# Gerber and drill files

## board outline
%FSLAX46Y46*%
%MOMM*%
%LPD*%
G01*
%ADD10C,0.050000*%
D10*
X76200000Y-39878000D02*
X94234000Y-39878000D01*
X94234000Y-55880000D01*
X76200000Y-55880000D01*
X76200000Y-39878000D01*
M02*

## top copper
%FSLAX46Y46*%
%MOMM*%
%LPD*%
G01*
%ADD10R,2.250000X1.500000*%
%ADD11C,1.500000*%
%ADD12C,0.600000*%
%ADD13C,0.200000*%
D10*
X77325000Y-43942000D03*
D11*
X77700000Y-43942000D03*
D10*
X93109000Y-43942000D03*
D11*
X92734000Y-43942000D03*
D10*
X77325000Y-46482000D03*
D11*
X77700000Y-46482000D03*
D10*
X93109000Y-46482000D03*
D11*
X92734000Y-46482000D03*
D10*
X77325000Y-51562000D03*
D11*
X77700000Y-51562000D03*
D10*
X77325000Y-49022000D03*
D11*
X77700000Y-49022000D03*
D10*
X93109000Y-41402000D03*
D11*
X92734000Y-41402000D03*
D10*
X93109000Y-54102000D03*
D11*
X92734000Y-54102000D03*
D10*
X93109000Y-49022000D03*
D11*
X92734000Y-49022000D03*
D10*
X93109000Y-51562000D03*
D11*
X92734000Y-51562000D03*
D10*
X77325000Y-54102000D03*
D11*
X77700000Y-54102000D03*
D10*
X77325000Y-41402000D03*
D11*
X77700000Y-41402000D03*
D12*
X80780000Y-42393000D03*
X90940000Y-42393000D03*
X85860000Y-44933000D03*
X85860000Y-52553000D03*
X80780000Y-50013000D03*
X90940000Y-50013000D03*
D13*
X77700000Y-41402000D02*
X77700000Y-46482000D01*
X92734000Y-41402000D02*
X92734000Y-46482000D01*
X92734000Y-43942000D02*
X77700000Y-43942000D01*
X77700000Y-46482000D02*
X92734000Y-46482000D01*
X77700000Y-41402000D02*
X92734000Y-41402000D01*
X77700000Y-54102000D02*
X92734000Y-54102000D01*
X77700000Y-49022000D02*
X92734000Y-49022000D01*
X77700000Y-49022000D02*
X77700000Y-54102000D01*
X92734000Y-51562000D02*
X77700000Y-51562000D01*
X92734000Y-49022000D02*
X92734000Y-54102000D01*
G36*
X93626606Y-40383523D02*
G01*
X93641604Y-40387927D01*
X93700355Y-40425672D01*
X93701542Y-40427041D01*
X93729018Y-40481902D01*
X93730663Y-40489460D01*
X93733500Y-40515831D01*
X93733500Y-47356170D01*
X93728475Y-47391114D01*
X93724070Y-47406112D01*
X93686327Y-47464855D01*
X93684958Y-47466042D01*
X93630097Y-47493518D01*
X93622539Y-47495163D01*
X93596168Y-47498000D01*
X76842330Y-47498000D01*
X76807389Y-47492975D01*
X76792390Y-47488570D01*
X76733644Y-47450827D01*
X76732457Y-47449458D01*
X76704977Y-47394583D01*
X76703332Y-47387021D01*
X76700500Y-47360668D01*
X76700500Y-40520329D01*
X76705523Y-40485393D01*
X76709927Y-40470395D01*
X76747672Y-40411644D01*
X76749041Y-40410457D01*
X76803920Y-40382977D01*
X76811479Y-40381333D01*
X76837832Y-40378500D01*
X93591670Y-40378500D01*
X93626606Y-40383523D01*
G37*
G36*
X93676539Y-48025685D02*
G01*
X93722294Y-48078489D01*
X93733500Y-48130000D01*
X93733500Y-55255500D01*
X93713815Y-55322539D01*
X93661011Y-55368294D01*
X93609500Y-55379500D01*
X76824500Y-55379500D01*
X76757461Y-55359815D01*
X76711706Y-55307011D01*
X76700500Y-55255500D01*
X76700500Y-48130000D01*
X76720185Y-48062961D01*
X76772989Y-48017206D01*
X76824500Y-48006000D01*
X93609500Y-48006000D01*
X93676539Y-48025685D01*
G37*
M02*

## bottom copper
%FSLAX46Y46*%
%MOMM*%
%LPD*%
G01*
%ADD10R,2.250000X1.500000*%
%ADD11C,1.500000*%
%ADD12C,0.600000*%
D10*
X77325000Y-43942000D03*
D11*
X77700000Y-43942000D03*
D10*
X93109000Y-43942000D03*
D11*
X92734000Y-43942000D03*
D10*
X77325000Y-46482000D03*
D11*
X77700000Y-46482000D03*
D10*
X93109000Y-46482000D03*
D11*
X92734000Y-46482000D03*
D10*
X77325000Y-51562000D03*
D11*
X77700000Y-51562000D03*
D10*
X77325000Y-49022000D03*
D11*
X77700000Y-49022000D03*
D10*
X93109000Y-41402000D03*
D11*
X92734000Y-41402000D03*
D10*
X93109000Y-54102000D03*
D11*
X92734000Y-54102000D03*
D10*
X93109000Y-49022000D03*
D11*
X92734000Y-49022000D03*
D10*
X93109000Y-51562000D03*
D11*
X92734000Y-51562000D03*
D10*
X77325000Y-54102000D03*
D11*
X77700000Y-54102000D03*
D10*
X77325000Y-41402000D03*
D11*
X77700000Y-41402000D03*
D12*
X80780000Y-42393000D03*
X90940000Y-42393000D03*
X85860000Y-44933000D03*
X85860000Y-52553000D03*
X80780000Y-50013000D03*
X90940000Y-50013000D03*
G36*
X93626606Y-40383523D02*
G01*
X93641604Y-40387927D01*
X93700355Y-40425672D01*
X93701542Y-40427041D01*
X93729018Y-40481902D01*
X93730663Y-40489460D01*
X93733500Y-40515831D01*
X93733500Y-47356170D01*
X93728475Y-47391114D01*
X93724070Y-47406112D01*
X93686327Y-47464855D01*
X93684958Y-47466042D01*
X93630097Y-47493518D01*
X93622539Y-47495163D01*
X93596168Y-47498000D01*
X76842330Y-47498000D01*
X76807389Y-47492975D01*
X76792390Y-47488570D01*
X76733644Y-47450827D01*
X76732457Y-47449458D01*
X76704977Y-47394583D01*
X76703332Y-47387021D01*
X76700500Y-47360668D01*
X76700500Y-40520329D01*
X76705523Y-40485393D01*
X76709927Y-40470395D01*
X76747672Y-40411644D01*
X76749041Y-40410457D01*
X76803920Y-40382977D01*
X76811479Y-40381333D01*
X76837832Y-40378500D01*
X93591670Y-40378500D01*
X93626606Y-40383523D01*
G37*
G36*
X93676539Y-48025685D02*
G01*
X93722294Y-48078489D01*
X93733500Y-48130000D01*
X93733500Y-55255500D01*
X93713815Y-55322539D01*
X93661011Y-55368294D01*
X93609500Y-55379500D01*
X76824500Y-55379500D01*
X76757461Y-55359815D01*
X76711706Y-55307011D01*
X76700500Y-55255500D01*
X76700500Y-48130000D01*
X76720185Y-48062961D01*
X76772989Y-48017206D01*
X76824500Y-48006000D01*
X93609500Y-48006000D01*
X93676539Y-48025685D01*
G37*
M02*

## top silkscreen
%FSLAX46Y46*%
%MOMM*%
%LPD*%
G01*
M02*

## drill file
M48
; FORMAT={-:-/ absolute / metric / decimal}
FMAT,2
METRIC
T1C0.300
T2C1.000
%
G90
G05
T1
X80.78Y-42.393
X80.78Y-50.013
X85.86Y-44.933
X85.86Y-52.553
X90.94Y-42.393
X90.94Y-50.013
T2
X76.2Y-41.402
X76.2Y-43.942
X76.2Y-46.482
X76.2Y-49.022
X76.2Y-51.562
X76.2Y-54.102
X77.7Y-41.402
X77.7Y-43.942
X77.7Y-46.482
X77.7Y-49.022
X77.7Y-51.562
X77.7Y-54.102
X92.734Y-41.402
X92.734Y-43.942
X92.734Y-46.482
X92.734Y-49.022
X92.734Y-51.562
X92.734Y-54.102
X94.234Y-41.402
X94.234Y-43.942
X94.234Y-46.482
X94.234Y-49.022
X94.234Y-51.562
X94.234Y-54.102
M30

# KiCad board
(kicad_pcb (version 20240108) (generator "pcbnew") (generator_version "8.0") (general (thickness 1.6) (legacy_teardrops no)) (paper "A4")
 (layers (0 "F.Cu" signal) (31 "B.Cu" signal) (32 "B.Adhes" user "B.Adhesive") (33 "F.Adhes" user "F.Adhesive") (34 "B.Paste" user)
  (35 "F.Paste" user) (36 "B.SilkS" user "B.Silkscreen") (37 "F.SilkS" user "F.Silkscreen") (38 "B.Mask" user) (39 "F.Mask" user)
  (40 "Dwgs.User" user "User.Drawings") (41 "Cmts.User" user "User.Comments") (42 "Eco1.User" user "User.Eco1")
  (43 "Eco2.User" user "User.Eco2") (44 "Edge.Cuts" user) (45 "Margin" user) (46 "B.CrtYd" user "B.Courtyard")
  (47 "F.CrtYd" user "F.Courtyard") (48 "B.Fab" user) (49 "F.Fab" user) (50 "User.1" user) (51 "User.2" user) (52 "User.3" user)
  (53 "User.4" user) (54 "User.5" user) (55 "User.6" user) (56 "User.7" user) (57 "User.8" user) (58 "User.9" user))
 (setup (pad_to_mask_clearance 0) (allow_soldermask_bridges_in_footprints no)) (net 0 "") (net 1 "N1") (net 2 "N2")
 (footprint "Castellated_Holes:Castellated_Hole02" (layer "F.Cu") (at 76.2 43.942)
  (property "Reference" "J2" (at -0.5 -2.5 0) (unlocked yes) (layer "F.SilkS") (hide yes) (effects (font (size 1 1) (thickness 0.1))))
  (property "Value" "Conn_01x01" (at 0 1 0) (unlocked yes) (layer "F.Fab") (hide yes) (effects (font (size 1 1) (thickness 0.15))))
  (pad "1" thru_hole rect (at 0 0) (size 2.25 1.5) (drill 1 (offset 1.125 0)) (layers "*.Cu" "*.Mask") (remove_unused_layers no)
   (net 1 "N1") (solder_mask_margin 0.04))
  (pad "1" thru_hole circle (at 1.5 0) (size 1.5 1.5) (drill 1) (layers "*.Cu" "*.Mask") (remove_unused_layers no) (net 1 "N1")
   (solder_mask_margin 0.04)))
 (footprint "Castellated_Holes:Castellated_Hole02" (layer "F.Cu") (at 94.234 43.942 180)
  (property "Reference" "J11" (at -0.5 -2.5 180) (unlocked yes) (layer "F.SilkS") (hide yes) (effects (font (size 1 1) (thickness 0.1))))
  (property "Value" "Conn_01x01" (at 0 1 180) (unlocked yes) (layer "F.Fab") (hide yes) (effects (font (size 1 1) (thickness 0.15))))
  (pad "1" thru_hole rect (at 0 0 180) (size 2.25 1.5) (drill 1 (offset 1.125 0)) (layers "*.Cu" "*.Mask") (remove_unused_layers no)
   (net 1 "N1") (solder_mask_margin 0.04))
  (pad "1" thru_hole circle (at 1.5 0 180) (size 1.5 1.5) (drill 1) (layers "*.Cu" "*.Mask") (remove_unused_layers no) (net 1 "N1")
   (solder_mask_margin 0.04)))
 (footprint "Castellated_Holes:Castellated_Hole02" (layer "F.Cu") (at 76.2 46.482)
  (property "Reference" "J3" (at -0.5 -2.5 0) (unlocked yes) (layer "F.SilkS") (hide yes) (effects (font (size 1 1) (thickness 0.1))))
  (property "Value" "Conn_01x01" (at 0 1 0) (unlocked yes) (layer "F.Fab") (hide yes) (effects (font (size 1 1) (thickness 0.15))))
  (pad "1" thru_hole rect (at 0 0) (size 2.25 1.5) (drill 1 (offset 1.125 0)) (layers "*.Cu" "*.Mask") (remove_unused_layers no)
   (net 1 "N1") (solder_mask_margin 0.04))
  (pad "1" thru_hole circle (at 1.5 0) (size 1.5 1.5) (drill 1) (layers "*.Cu" "*.Mask") (remove_unused_layers no) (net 1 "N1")
   (solder_mask_margin 0.04)))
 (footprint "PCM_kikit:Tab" (layer "F.Cu") (at 92.964 39.624 -90)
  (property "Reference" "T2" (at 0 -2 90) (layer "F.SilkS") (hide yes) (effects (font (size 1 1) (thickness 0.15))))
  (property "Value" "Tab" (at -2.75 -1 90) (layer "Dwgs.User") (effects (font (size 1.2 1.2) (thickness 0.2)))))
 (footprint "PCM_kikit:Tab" (layer "F.Cu") (at 77.47 39.624 -90)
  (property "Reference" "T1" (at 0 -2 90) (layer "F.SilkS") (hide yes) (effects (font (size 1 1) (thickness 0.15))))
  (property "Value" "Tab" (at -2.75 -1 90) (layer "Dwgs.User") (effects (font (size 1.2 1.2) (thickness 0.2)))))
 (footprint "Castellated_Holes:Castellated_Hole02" (layer "F.Cu") (at 94.234 46.482 180)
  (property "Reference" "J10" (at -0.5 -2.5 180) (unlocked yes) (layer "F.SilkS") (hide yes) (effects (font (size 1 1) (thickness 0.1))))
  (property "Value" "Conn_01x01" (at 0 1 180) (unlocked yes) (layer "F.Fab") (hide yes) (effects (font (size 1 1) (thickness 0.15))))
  (pad "1" thru_hole rect (at 0 0 180) (size 2.25 1.5) (drill 1 (offset 1.125 0)) (layers "*.Cu" "*.Mask") (remove_unused_layers no)
   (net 1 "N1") (solder_mask_margin 0.04))
  (pad "1" thru_hole circle (at 1.5 0 180) (size 1.5 1.5) (drill 1) (layers "*.Cu" "*.Mask") (remove_unused_layers no) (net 1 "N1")
   (solder_mask_margin 0.04)))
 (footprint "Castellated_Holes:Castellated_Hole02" (layer "F.Cu") (at 76.2 51.562)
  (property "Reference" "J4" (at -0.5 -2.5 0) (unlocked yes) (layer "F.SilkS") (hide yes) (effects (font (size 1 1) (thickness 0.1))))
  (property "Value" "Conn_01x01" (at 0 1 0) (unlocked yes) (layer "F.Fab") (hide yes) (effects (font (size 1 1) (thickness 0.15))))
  (pad "1" thru_hole rect (at 0 0) (size 2.25 1.5) (drill 1 (offset 1.125 0)) (layers "*.Cu" "*.Mask") (remove_unused_layers no)
   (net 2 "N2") (solder_mask_margin 0.04))
  (pad "1" thru_hole circle (at 1.5 0) (size 1.5 1.5) (drill 1) (layers "*.Cu" "*.Mask") (remove_unused_layers no) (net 2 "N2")
   (solder_mask_margin 0.04)))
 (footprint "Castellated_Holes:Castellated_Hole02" (layer "F.Cu") (at 76.2 49.022)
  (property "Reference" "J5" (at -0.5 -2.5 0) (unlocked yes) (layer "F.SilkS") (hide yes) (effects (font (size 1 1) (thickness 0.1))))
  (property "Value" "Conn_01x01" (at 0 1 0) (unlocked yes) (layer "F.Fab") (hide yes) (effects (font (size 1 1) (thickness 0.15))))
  (pad "1" thru_hole rect (at 0 0) (size 2.25 1.5) (drill 1 (offset 1.125 0)) (layers "*.Cu" "*.Mask") (remove_unused_layers no)
   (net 2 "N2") (solder_mask_margin 0.04))
  (pad "1" thru_hole circle (at 1.5 0) (size 1.5 1.5) (drill 1) (layers "*.Cu" "*.Mask") (remove_unused_layers no) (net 2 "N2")
   (solder_mask_margin 0.04)))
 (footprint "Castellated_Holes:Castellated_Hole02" (layer "F.Cu") (at 94.234 41.402 180)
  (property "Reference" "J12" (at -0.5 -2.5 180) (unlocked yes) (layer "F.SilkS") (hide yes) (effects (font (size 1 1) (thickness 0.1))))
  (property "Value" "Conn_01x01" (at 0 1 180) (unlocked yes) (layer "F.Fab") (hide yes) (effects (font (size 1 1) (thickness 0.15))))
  (pad "1" thru_hole rect (at 0 0 180) (size 2.25 1.5) (drill 1 (offset 1.125 0)) (layers "*.Cu" "*.Mask") (remove_unused_layers no)
   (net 1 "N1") (solder_mask_margin 0.04))
  (pad "1" thru_hole circle (at 1.5 0 180) (size 1.5 1.5) (drill 1) (layers "*.Cu" "*.Mask") (remove_unused_layers no) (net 1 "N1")
   (solder_mask_margin 0.04)))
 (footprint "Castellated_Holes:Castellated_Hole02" (layer "F.Cu") (at 94.234 54.102 180)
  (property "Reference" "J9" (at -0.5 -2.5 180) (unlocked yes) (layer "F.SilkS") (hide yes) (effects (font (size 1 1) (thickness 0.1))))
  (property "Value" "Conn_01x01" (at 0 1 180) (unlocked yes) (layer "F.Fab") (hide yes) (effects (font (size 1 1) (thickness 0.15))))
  (pad "1" thru_hole rect (at 0 0 180) (size 2.25 1.5) (drill 1 (offset 1.125 0)) (layers "*.Cu" "*.Mask") (remove_unused_layers no)
   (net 2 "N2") (solder_mask_margin 0.04))
  (pad "1" thru_hole circle (at 1.5 0 180) (size 1.5 1.5) (drill 1) (layers "*.Cu" "*.Mask") (remove_unused_layers no) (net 2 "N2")
   (solder_mask_margin 0.04)))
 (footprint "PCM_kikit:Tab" (layer "F.Cu") (at 77.47 56.134 90)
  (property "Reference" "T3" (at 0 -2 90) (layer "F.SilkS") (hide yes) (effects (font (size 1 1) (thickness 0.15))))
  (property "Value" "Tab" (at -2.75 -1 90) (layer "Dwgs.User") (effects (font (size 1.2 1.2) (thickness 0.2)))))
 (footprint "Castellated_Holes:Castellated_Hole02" (layer "F.Cu") (at 94.234 49.022 180)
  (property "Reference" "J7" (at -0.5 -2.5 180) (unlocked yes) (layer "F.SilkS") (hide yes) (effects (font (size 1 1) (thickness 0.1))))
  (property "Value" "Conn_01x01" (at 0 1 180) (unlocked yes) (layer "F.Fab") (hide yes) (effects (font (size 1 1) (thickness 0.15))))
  (pad "1" thru_hole rect (at 0 0 180) (size 2.25 1.5) (drill 1 (offset 1.125 0)) (layers "*.Cu" "*.Mask") (remove_unused_layers no)
   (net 2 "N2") (solder_mask_margin 0.04))
  (pad "1" thru_hole circle (at 1.5 0 180) (size 1.5 1.5) (drill 1) (layers "*.Cu" "*.Mask") (remove_unused_layers no) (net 2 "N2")
   (solder_mask_margin 0.04)))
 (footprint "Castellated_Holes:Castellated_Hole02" (layer "F.Cu") (at 94.234 51.562 180)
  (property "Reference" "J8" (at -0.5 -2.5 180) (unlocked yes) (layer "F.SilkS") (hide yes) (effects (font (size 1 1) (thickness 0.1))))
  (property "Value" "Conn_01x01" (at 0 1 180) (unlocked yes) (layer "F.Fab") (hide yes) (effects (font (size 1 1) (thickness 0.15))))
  (pad "1" thru_hole rect (at 0 0 180) (size 2.25 1.5) (drill 1 (offset 1.125 0)) (layers "*.Cu" "*.Mask") (remove_unused_layers no)
   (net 2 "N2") (solder_mask_margin 0.04))
  (pad "1" thru_hole circle (at 1.5 0 180) (size 1.5 1.5) (drill 1) (layers "*.Cu" "*.Mask") (remove_unused_layers no) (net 2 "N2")
   (solder_mask_margin 0.04)))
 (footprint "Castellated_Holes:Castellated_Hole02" (layer "F.Cu") (at 76.2 54.102)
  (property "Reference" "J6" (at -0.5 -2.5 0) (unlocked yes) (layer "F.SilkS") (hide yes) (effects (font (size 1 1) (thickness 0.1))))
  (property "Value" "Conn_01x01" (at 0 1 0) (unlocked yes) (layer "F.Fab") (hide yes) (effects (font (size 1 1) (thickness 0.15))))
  (pad "1" thru_hole rect (at 0 0) (size 2.25 1.5) (drill 1 (offset 1.125 0)) (layers "*.Cu" "*.Mask") (remove_unused_layers no)
   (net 2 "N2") (solder_mask_margin 0.04))
  (pad "1" thru_hole circle (at 1.5 0) (size 1.5 1.5) (drill 1) (layers "*.Cu" "*.Mask") (remove_unused_layers no) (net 2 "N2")
   (solder_mask_margin 0.04)))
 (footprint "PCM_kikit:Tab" (layer "F.Cu") (at 92.964 56.154 90)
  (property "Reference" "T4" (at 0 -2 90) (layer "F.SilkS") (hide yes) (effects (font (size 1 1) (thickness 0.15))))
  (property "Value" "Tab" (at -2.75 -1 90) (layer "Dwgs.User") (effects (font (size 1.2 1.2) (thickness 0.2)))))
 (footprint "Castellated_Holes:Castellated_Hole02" (layer "F.Cu") (at 76.2 41.402)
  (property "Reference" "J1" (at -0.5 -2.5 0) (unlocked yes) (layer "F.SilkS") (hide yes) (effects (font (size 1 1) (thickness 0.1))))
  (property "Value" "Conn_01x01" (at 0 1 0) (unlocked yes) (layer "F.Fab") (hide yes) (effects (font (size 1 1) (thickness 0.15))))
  (pad "1" thru_hole rect (at 0 0) (size 2.25 1.5) (drill 1 (offset 1.125 0)) (layers "*.Cu" "*.Mask") (remove_unused_layers no)
   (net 1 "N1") (solder_mask_margin 0.04))
  (pad "1" thru_hole circle (at 1.5 0) (size 1.5 1.5) (drill 1) (layers "*.Cu" "*.Mask") (remove_unused_layers no) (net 1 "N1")
   (solder_mask_margin 0.04)))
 (gr_rect (start 76.2 39.878) (end 94.234 55.88) (stroke (width 0.05) (type default)) (fill none) (layer "Edge.Cuts"))
 (segment (start 77.7 41.402) (end 77.7 46.482) (width 0.2) (layer "F.Cu") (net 1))
 (segment (start 92.734 41.402) (end 92.734 46.482) (width 0.2) (layer "F.Cu") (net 1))
 (segment (start 92.734 43.942) (end 77.7 43.942) (width 0.2) (layer "F.Cu") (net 1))
 (segment (start 77.7 46.482) (end 92.734 46.482) (width 0.2) (layer "F.Cu") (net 1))
 (segment (start 77.7 41.402) (end 92.734 41.402) (width 0.2) (layer "F.Cu") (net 1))
 (via (at 80.78 42.393) (size 0.6) (drill 0.3) (layers "F.Cu" "B.Cu") (free yes) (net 1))
 (via (at 90.94 42.393) (size 0.6) (drill 0.3) (layers "F.Cu" "B.Cu") (free yes) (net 1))
 (via (at 85.86 44.933) (size 0.6) (drill 0.3) (layers "F.Cu" "B.Cu") (free yes) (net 1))
 (segment (start 77.7 54.102) (end 92.734 54.102) (width 0.2) (layer "F.Cu") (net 2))
 (segment (start 77.7 49.022) (end 92.734 49.022) (width 0.2) (layer "F.Cu") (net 2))
 (segment (start 77.7 49.022) (end 77.7 54.102) (width 0.2) (layer "F.Cu") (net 2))
 (segment (start 92.734 51.562) (end 77.7 51.562) (width 0.2) (layer "F.Cu") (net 2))
 (segment (start 92.734 49.022) (end 92.734 54.102) (width 0.2) (layer "F.Cu") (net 2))
 (via (at 85.86 52.553) (size 0.6) (drill 0.3) (layers "F.Cu" "B.Cu") (free yes) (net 2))
 (via (at 80.78 50.013) (size 0.6) (drill 0.3) (layers "F.Cu" "B.Cu") (free yes) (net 2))
 (via (at 90.94 50.013) (size 0.6) (drill 0.3) (layers "F.Cu" "B.Cu") (free yes) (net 2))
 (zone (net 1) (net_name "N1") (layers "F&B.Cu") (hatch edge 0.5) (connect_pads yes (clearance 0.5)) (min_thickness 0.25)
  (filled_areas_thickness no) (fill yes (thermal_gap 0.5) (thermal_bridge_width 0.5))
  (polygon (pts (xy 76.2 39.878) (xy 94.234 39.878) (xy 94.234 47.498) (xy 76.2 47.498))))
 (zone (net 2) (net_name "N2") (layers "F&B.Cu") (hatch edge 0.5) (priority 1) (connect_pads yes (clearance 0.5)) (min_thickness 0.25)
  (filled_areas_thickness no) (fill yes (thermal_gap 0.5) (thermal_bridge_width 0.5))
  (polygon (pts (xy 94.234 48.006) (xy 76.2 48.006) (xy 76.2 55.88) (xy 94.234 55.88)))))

